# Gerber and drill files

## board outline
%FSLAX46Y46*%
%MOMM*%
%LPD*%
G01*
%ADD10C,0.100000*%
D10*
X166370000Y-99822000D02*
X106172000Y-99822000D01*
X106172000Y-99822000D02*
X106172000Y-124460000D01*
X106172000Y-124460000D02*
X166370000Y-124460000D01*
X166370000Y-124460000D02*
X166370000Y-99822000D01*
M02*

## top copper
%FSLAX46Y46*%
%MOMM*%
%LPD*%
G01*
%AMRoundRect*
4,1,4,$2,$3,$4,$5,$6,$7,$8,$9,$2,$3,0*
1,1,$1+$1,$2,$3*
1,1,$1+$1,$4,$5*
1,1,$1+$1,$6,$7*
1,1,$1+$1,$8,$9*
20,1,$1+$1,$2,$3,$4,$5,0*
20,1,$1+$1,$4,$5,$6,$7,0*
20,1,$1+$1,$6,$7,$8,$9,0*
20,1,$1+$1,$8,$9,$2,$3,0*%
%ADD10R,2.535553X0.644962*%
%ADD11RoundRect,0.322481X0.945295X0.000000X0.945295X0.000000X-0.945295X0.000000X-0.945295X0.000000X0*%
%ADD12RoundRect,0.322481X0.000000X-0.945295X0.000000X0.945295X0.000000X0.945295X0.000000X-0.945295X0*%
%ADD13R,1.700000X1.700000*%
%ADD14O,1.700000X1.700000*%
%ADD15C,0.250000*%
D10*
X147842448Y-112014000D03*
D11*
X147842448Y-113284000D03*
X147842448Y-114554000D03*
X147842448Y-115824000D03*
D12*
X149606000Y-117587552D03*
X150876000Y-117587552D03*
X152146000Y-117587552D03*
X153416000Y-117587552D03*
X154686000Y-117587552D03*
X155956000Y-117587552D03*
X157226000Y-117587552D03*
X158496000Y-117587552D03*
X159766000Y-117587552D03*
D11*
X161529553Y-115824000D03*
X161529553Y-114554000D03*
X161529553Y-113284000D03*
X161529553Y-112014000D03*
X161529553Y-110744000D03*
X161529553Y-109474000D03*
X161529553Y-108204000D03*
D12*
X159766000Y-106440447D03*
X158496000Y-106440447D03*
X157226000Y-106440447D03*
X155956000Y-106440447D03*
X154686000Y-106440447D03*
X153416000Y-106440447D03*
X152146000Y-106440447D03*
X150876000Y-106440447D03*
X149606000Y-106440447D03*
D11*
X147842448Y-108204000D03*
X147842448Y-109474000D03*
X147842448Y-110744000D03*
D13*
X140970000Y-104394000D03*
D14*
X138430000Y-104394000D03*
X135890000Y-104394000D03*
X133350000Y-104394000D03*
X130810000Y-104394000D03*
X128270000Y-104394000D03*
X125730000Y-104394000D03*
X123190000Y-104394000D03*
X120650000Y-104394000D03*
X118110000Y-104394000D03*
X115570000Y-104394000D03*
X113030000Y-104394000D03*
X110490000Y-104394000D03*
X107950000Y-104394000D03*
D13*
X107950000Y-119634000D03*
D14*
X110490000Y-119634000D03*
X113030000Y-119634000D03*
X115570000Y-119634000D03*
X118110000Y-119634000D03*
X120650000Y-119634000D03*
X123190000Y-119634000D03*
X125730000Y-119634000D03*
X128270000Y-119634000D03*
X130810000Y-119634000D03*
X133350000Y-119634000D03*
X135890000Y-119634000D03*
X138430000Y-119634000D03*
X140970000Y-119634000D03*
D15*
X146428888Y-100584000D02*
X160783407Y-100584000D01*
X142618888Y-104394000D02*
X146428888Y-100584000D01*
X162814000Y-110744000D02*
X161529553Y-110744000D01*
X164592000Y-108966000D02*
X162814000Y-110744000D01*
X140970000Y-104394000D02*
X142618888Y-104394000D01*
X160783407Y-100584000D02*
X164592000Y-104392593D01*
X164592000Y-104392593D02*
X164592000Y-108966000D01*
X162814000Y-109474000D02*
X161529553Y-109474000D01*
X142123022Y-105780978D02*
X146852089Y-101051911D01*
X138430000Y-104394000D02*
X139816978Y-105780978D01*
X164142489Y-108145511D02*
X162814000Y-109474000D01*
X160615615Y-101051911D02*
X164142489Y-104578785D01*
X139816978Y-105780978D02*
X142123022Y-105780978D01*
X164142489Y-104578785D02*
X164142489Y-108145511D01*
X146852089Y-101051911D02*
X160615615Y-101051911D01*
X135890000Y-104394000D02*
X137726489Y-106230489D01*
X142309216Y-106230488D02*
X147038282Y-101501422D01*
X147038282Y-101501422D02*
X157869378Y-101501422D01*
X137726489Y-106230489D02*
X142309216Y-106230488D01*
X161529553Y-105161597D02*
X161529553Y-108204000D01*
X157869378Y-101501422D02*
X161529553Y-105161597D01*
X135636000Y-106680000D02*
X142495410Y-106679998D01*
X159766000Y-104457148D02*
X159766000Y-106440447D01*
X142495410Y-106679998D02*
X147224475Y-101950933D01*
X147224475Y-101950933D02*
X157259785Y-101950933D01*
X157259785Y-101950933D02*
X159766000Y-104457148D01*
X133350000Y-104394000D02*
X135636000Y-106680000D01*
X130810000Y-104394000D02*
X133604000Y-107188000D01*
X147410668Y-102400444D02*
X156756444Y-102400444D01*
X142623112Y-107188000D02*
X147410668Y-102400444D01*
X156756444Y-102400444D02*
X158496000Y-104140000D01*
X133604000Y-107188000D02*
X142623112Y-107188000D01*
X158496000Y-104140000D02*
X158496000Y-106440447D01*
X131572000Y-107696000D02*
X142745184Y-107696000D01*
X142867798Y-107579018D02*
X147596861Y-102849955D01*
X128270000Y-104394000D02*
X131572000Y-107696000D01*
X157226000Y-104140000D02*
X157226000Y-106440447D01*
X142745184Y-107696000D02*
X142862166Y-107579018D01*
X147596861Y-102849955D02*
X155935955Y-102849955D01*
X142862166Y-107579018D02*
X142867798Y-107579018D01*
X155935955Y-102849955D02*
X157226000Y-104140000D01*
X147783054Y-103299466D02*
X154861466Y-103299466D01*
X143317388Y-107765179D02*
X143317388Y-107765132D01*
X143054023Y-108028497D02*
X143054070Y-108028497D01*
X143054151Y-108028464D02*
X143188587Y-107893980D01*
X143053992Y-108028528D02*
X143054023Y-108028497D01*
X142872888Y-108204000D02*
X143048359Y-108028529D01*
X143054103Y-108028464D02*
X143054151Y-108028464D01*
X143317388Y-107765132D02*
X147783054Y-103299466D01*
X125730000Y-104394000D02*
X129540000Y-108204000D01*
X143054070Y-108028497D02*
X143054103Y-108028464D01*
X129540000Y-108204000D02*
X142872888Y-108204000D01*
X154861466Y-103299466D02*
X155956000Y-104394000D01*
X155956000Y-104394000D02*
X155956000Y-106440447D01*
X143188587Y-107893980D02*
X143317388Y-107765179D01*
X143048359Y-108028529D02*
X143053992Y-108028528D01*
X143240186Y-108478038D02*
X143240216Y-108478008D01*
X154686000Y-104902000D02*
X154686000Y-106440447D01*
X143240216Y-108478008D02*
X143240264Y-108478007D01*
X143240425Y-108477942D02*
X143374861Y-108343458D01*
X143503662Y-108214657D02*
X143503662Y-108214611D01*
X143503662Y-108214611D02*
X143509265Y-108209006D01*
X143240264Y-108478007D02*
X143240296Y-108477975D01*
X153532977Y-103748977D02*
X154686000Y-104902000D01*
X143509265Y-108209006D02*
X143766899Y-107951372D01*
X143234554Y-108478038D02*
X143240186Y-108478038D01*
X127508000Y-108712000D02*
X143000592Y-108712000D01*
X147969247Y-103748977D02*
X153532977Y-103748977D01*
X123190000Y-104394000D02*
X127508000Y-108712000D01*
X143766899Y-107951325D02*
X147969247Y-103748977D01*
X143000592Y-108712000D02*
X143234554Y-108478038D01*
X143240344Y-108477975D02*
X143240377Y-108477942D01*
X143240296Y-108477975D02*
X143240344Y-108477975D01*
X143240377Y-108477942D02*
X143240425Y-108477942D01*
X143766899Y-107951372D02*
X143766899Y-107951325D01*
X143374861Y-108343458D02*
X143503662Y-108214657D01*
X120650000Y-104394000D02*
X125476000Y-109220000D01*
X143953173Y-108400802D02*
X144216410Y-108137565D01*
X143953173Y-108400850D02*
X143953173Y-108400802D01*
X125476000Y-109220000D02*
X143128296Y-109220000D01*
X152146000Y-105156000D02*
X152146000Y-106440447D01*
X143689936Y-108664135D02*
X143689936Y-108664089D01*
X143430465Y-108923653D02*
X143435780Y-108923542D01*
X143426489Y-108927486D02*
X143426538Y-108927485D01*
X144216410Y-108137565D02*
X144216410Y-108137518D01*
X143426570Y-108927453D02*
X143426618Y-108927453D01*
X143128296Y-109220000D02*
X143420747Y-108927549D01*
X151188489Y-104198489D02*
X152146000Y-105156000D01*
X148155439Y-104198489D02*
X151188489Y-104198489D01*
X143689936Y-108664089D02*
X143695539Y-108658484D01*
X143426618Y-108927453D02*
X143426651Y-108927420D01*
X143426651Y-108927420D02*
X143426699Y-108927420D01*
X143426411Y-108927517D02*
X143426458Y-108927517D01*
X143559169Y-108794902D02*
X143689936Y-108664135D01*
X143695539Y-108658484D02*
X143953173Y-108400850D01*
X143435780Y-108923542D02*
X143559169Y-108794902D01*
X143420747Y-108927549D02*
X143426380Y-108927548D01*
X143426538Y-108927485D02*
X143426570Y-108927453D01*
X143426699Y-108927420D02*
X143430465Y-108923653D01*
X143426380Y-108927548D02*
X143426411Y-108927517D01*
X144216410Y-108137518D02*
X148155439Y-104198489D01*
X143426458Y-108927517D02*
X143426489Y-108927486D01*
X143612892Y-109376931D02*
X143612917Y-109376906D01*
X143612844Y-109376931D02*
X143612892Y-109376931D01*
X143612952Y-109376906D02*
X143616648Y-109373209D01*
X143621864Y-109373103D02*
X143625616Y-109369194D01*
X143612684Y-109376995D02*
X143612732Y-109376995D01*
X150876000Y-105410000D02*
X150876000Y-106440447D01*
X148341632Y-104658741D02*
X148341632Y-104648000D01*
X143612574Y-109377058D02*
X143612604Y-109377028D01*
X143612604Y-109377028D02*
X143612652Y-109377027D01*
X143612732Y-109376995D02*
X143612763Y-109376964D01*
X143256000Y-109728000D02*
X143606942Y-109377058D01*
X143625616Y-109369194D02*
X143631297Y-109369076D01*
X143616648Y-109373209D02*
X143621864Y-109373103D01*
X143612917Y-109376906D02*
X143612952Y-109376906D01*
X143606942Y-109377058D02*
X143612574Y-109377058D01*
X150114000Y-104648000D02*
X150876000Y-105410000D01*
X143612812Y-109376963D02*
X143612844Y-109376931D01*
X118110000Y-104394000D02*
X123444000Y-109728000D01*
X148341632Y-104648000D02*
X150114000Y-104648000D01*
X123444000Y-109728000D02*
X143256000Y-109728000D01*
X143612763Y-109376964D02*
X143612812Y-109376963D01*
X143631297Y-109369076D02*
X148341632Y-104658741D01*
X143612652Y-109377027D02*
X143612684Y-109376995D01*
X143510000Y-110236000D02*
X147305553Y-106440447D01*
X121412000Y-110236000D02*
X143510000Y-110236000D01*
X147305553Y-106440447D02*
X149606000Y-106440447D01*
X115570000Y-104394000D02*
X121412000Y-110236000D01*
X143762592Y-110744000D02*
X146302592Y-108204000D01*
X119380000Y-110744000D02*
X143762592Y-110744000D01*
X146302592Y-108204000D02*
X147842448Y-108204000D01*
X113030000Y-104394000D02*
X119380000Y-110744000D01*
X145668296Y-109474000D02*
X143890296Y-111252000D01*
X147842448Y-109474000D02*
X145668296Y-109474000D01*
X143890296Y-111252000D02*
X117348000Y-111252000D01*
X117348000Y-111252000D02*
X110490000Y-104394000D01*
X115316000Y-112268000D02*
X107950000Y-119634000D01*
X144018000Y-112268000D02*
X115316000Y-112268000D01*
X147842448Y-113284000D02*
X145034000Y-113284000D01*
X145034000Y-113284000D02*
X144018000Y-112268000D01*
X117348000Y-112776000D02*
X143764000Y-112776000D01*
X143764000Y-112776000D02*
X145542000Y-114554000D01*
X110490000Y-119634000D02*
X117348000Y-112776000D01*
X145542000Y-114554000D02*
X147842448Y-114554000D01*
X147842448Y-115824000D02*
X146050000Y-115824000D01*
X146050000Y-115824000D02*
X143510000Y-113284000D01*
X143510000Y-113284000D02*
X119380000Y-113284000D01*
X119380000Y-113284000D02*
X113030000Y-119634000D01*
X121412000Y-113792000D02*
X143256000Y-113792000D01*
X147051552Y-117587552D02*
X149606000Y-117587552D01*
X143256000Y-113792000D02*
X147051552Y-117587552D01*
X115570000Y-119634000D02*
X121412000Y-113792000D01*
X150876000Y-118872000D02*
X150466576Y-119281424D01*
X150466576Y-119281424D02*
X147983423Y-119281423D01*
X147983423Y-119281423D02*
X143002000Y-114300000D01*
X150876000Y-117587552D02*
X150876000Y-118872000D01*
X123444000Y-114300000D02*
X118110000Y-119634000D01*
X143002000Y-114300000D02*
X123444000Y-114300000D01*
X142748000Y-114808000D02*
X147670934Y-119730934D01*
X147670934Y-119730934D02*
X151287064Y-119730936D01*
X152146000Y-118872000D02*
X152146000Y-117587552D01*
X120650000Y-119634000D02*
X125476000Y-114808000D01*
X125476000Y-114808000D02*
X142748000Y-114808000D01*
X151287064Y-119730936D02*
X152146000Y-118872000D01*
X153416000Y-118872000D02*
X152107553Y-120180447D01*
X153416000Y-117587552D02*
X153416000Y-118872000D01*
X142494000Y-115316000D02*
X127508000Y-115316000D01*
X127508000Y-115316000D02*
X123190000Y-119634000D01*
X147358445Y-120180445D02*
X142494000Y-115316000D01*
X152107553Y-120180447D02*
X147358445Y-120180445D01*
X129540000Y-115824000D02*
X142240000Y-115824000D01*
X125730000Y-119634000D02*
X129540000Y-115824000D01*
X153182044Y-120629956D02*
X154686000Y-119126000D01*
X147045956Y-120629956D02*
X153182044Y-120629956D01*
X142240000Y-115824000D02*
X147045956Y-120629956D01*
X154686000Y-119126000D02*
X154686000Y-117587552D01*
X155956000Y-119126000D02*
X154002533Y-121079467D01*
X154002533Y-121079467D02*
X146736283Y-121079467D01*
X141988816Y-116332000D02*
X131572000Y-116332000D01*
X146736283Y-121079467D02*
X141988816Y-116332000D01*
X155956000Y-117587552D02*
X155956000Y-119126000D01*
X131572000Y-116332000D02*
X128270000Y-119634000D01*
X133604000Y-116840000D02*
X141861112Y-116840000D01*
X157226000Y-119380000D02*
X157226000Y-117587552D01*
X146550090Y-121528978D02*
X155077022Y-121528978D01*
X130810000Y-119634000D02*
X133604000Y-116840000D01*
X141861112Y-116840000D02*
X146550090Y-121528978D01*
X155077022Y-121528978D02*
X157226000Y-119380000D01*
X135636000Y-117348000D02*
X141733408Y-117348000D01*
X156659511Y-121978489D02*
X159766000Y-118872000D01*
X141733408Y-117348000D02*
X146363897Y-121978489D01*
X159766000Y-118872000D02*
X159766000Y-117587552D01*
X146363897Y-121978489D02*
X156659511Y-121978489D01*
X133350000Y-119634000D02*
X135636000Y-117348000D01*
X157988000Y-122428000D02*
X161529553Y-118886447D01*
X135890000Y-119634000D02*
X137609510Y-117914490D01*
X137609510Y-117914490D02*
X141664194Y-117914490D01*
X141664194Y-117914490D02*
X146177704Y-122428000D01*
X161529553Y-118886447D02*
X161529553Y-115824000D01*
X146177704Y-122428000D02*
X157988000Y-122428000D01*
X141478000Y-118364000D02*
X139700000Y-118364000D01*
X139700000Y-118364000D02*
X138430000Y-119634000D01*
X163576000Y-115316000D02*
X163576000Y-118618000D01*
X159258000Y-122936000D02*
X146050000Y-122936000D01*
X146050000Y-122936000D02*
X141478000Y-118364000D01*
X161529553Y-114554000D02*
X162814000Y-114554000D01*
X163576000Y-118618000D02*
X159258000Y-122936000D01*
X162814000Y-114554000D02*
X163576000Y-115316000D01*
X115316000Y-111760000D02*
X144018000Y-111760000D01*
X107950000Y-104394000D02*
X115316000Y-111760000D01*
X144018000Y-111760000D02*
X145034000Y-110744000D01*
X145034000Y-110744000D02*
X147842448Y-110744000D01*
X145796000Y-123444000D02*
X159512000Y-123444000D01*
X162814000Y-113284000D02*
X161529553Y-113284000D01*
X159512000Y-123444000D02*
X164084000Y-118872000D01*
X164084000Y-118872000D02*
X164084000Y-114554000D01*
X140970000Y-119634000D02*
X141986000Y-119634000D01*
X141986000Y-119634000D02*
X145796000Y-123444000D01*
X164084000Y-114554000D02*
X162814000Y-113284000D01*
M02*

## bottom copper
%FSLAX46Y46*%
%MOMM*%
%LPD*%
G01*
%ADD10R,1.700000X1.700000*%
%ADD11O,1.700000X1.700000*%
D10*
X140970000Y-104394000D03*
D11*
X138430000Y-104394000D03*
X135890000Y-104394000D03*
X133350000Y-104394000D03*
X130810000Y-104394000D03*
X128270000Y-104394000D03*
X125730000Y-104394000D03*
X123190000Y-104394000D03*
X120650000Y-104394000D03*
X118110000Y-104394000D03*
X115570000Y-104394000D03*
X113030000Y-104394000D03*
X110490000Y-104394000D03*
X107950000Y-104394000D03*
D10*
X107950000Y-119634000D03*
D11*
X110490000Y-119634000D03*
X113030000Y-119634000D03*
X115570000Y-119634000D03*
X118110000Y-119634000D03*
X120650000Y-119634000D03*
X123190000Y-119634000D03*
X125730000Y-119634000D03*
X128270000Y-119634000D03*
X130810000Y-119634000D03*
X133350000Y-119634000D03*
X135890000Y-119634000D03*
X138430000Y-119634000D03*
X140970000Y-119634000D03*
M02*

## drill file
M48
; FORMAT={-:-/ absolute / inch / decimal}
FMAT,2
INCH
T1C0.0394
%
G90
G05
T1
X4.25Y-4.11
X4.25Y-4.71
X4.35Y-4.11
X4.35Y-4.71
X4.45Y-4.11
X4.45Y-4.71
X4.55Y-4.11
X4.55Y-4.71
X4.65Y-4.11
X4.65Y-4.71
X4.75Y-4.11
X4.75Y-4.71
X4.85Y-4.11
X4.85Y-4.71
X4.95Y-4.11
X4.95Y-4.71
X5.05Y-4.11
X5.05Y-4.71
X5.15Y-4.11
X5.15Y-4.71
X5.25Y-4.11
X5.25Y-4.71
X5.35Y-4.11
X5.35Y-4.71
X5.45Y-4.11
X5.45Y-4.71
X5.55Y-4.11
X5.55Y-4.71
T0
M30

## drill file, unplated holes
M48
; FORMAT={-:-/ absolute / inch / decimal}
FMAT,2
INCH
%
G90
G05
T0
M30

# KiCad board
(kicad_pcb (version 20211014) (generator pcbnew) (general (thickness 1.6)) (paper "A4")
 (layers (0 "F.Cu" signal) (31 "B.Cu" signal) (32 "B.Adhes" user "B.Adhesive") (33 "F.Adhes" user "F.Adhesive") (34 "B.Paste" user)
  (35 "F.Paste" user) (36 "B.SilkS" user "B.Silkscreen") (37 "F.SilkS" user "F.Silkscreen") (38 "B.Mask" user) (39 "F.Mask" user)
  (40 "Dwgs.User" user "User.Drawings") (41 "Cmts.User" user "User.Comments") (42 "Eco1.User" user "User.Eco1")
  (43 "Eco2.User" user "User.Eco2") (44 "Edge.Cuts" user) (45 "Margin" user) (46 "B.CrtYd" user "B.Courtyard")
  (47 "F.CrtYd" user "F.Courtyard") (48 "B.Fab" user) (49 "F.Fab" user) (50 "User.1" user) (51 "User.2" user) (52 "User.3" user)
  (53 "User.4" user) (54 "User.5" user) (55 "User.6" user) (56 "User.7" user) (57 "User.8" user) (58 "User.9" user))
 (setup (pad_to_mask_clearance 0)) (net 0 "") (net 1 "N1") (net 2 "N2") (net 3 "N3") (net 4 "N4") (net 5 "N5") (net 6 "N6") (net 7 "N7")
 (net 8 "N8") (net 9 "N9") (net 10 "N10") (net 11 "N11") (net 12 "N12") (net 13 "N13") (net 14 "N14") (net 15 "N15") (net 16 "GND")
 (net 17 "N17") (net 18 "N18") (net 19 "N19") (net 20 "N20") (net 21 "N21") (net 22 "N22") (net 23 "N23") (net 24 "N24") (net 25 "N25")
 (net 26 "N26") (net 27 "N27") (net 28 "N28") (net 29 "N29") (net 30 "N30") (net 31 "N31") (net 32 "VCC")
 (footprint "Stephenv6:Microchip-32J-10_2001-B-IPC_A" (layer "F.Cu") (at 154.686 112.014 90)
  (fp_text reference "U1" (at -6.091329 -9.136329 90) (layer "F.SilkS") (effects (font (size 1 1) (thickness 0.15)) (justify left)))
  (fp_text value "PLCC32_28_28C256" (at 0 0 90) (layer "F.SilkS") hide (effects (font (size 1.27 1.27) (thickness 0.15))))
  (pad "1" smd rect (at 0 -6.843552 90) (size 0.644962 2.535553) (layers "F.Cu" "F.Paste" "F.Mask") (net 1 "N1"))
  (pad "2" smd roundrect (at -1.27 -6.843552 90) (size 0.644962 2.535553) (layers "F.Cu" "F.Paste" "F.Mask") (roundrect_rratio 0.5)
   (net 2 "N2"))
  (pad "3" smd roundrect (at -2.54 -6.843552 90) (size 0.644962 2.535553) (layers "F.Cu" "F.Paste" "F.Mask") (roundrect_rratio 0.5)
   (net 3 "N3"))
  (pad "4" smd roundrect (at -3.81 -6.843552 90) (size 0.644962 2.535553) (layers "F.Cu" "F.Paste" "F.Mask") (roundrect_rratio 0.5)
   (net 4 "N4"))
  (pad "5" smd roundrect (at -5.573552 -5.08 90) (size 2.535553 0.644962) (layers "F.Cu" "F.Paste" "F.Mask") (roundrect_rratio 0.5)
   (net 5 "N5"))
  (pad "6" smd roundrect (at -5.573552 -3.81 90) (size 2.535553 0.644962) (layers "F.Cu" "F.Paste" "F.Mask") (roundrect_rratio 0.5)
   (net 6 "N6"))
  (pad "7" smd roundrect (at -5.573552 -2.54 90) (size 2.535553 0.644962) (layers "F.Cu" "F.Paste" "F.Mask") (roundrect_rratio 0.5)
   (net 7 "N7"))
  (pad "8" smd roundrect (at -5.573552 -1.27 90) (size 2.535553 0.644962) (layers "F.Cu" "F.Paste" "F.Mask") (roundrect_rratio 0.5)
   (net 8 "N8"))
  (pad "9" smd roundrect (at -5.573552 0 90) (size 2.535553 0.644962) (layers "F.Cu" "F.Paste" "F.Mask") (roundrect_rratio 0.5) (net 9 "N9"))
  (pad "10" smd roundrect (at -5.573552 1.27 90) (size 2.535553 0.644962) (layers "F.Cu" "F.Paste" "F.Mask") (roundrect_rratio 0.5)
   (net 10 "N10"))
  (pad "11" smd roundrect (at -5.573552 2.54 90) (size 2.535553 0.644962) (layers "F.Cu" "F.Paste" "F.Mask") (roundrect_rratio 0.5)
   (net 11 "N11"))
  (pad "12" smd roundrect (at -5.573552 3.81 90) (size 2.535553 0.644962) (layers "F.Cu" "F.Paste" "F.Mask") (roundrect_rratio 0.5)
   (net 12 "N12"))
  (pad "13" smd roundrect (at -5.573552 5.08 90) (size 2.535553 0.644962) (layers "F.Cu" "F.Paste" "F.Mask") (roundrect_rratio 0.5)
   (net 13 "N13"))
  (pad "14" smd roundrect (at -3.81 6.843553 90) (size 0.644962 2.535553) (layers "F.Cu" "F.Paste" "F.Mask") (roundrect_rratio 0.5)
   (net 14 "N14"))
  (pad "15" smd roundrect (at -2.54 6.843553 90) (size 0.644962 2.535553) (layers "F.Cu" "F.Paste" "F.Mask") (roundrect_rratio 0.5)
   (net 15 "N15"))
  (pad "16" smd roundrect (at -1.27 6.843553 90) (size 0.644962 2.535553) (layers "F.Cu" "F.Paste" "F.Mask") (roundrect_rratio 0.5)
   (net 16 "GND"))
  (pad "17" smd roundrect (at 0 6.843553 90) (size 0.644962 2.535553) (layers "F.Cu" "F.Paste" "F.Mask") (roundrect_rratio 0.5)
   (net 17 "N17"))
  (pad "18" smd roundrect (at 1.27 6.843553 90) (size 0.644962 2.535553) (layers "F.Cu" "F.Paste" "F.Mask") (roundrect_rratio 0.5)
   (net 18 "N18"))
  (pad "19" smd roundrect (at 2.54 6.843553 90) (size 0.644962 2.535553) (layers "F.Cu" "F.Paste" "F.Mask") (roundrect_rratio 0.5)
   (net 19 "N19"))
  (pad "20" smd roundrect (at 3.81 6.843553 90) (size 0.644962 2.535553) (layers "F.Cu" "F.Paste" "F.Mask") (roundrect_rratio 0.5)
   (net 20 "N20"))
  (pad "21" smd roundrect (at 5.573553 5.08 90) (size 2.535553 0.644962) (layers "F.Cu" "F.Paste" "F.Mask") (roundrect_rratio 0.5)
   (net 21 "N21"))
  (pad "22" smd roundrect (at 5.573553 3.81 90) (size 2.535553 0.644962) (layers "F.Cu" "F.Paste" "F.Mask") (roundrect_rratio 0.5)
   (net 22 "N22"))
  (pad "23" smd roundrect (at 5.573553 2.54 90) (size 2.535553 0.644962) (layers "F.Cu" "F.Paste" "F.Mask") (roundrect_rratio 0.5)
   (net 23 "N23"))
  (pad "24" smd roundrect (at 5.573553 1.27 90) (size 2.535553 0.644962) (layers "F.Cu" "F.Paste" "F.Mask") (roundrect_rratio 0.5)
   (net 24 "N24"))
  (pad "25" smd roundrect (at 5.573553 0 90) (size 2.535553 0.644962) (layers "F.Cu" "F.Paste" "F.Mask") (roundrect_rratio 0.5)
   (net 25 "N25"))
  (pad "26" smd roundrect (at 5.573553 -1.27 90) (size 2.535553 0.644962) (layers "F.Cu" "F.Paste" "F.Mask") (roundrect_rratio 0.5)
   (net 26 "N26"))
  (pad "27" smd roundrect (at 5.573553 -2.54 90) (size 2.535553 0.644962) (layers "F.Cu" "F.Paste" "F.Mask") (roundrect_rratio 0.5)
   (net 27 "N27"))
  (pad "28" smd roundrect (at 5.573553 -3.81 90) (size 2.535553 0.644962) (layers "F.Cu" "F.Paste" "F.Mask") (roundrect_rratio 0.5)
   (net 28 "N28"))
  (pad "29" smd roundrect (at 5.573553 -5.08 90) (size 2.535553 0.644962) (layers "F.Cu" "F.Paste" "F.Mask") (roundrect_rratio 0.5)
   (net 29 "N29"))
  (pad "30" smd roundrect (at 3.81 -6.843552 90) (size 0.644962 2.535553) (layers "F.Cu" "F.Paste" "F.Mask") (roundrect_rratio 0.5)
   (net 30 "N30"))
  (pad "31" smd roundrect (at 2.54 -6.843552 90) (size 0.644962 2.535553) (layers "F.Cu" "F.Paste" "F.Mask") (roundrect_rratio 0.5)
   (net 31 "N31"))
  (pad "32" smd roundrect (at 1.27 -6.843552 90) (size 0.644962 2.535553) (layers "F.Cu" "F.Paste" "F.Mask") (roundrect_rratio 0.5)
   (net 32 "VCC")))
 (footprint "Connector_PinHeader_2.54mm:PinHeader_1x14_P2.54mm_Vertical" (layer "B.Cu") (at 140.97 104.394 90)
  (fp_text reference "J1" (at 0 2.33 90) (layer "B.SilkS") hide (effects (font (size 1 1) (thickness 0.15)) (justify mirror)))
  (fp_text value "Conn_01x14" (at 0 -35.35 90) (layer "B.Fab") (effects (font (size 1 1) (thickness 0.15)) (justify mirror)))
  (pad "1" thru_hole rect locked (at 0 0 90) (size 1.7 1.7) (drill 1) (layers *.Cu *.Mask) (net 18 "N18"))
  (pad "2" thru_hole oval locked (at 0 -2.54 90) (size 1.7 1.7) (drill 1) (layers *.Cu *.Mask) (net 19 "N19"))
  (pad "3" thru_hole oval locked (at 0 -5.08 90) (size 1.7 1.7) (drill 1) (layers *.Cu *.Mask) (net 20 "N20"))
  (pad "4" thru_hole oval locked (at 0 -7.62 90) (size 1.7 1.7) (drill 1) (layers *.Cu *.Mask) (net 21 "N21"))
  (pad "5" thru_hole oval locked (at 0 -10.16 90) (size 1.7 1.7) (drill 1) (layers *.Cu *.Mask) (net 22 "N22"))
  (pad "6" thru_hole oval locked (at 0 -12.7 90) (size 1.7 1.7) (drill 1) (layers *.Cu *.Mask) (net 23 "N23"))
  (pad "7" thru_hole oval locked (at 0 -15.24 90) (size 1.7 1.7) (drill 1) (layers *.Cu *.Mask) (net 24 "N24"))
  (pad "8" thru_hole oval locked (at 0 -17.78 90) (size 1.7 1.7) (drill 1) (layers *.Cu *.Mask) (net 25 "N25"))
  (pad "9" thru_hole oval locked (at 0 -20.32 90) (size 1.7 1.7) (drill 1) (layers *.Cu *.Mask) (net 27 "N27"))
  (pad "10" thru_hole oval locked (at 0 -22.86 90) (size 1.7 1.7) (drill 1) (layers *.Cu *.Mask) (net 28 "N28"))
  (pad "11" thru_hole oval locked (at 0 -25.4 90) (size 1.7 1.7) (drill 1) (layers *.Cu *.Mask) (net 29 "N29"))
  (pad "12" thru_hole oval locked (at 0 -27.94 90) (size 1.7 1.7) (drill 1) (layers *.Cu *.Mask) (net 30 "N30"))
  (pad "13" thru_hole oval locked (at 0 -30.48 90) (size 1.7 1.7) (drill 1) (layers *.Cu *.Mask) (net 31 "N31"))
  (pad "14" thru_hole oval locked (at 0 -33.02 90) (size 1.7 1.7) (drill 1) (layers *.Cu *.Mask) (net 32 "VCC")))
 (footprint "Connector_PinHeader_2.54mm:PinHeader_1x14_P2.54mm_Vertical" (layer "B.Cu") (at 107.95 119.634 -90)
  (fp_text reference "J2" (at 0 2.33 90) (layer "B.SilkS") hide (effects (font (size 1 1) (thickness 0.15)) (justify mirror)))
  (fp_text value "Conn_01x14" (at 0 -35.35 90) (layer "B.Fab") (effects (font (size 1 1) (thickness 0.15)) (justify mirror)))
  (pad "1" thru_hole rect locked (at 0 0 270) (size 1.7 1.7) (drill 1) (layers *.Cu *.Mask) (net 2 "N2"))
  (pad "2" thru_hole oval locked (at 0 -2.54 270) (size 1.7 1.7) (drill 1) (layers *.Cu *.Mask) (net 3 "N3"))
  (pad "3" thru_hole oval locked (at 0 -5.08 270) (size 1.7 1.7) (drill 1) (layers *.Cu *.Mask) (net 4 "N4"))
  (pad "4" thru_hole oval locked (at 0 -7.62 270) (size 1.7 1.7) (drill 1) (layers *.Cu *.Mask) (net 5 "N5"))
  (pad "5" thru_hole oval locked (at 0 -10.16 270) (size 1.7 1.7) (drill 1) (layers *.Cu *.Mask) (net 6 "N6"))
  (pad "6" thru_hole oval locked (at 0 -12.7 270) (size 1.7 1.7) (drill 1) (layers *.Cu *.Mask) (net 7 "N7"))
  (pad "7" thru_hole oval locked (at 0 -15.24 270) (size 1.7 1.7) (drill 1) (layers *.Cu *.Mask) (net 8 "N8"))
  (pad "8" thru_hole oval locked (at 0 -17.78 270) (size 1.7 1.7) (drill 1) (layers *.Cu *.Mask) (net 9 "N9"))
  (pad "9" thru_hole oval locked (at 0 -20.32 270) (size 1.7 1.7) (drill 1) (layers *.Cu *.Mask) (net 10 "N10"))
  (pad "10" thru_hole oval locked (at 0 -22.86 270) (size 1.7 1.7) (drill 1) (layers *.Cu *.Mask) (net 11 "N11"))
  (pad "11" thru_hole oval locked (at 0 -25.4 270) (size 1.7 1.7) (drill 1) (layers *.Cu *.Mask) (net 13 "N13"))
  (pad "12" thru_hole oval locked (at 0 -27.94 270) (size 1.7 1.7) (drill 1) (layers *.Cu *.Mask) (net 14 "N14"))
  (pad "13" thru_hole oval locked (at 0 -30.48 270) (size 1.7 1.7) (drill 1) (layers *.Cu *.Mask) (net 15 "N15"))
  (pad "14" thru_hole oval locked (at 0 -33.02 270) (size 1.7 1.7) (drill 1) (layers *.Cu *.Mask) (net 16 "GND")))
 (gr_rect (start 166.37 99.822) (end 106.172 124.46) (layer "Edge.Cuts") (width 0.1) (fill none))
 (segment (start 146.428888 100.584) (end 160.783407 100.584) (width 0.25) (layer "F.Cu") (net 18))
 (segment (start 142.618888 104.394) (end 146.428888 100.584) (width 0.25) (layer "F.Cu") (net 18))
 (segment (start 162.814 110.744) (end 161.529553 110.744) (width 0.25) (layer "F.Cu") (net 18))
 (segment (start 164.592 108.966) (end 162.814 110.744) (width 0.25) (layer "F.Cu") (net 18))
 (segment (start 140.97 104.394) (end 142.618888 104.394) (width 0.25) (layer "F.Cu") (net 18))
 (segment (start 160.783407 100.584) (end 164.592 104.392593) (width 0.25) (layer "F.Cu") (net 18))
 (segment (start 164.592 104.392593) (end 164.592 108.966) (width 0.25) (layer "F.Cu") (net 18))
 (segment (start 162.814 109.474) (end 161.529553 109.474) (width 0.25) (layer "F.Cu") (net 19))
 (segment (start 142.123022 105.780978) (end 146.852089 101.051911) (width 0.25) (layer "F.Cu") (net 19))
 (segment (start 138.43 104.394) (end 139.816978 105.780978) (width 0.25) (layer "F.Cu") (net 19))
 (segment (start 164.142489 108.145511) (end 162.814 109.474) (width 0.25) (layer "F.Cu") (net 19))
 (segment (start 160.615615 101.051911) (end 164.142489 104.578785) (width 0.25) (layer "F.Cu") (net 19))
 (segment (start 139.816978 105.780978) (end 142.123022 105.780978) (width 0.25) (layer "F.Cu") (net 19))
 (segment (start 164.142489 104.578785) (end 164.142489 108.145511) (width 0.25) (layer "F.Cu") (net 19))
 (segment (start 146.852089 101.051911) (end 160.615615 101.051911) (width 0.25) (layer "F.Cu") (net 19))
 (segment (start 135.89 104.394) (end 137.726489 106.230489) (width 0.25) (layer "F.Cu") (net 20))
 (segment (start 142.309216 106.230488) (end 147.038282 101.501422) (width 0.25) (layer "F.Cu") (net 20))
 (segment (start 147.038282 101.501422) (end 157.869378 101.501422) (width 0.25) (layer "F.Cu") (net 20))
 (segment (start 137.726489 106.230489) (end 142.309216 106.230488) (width 0.25) (layer "F.Cu") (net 20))
 (segment (start 161.529553 105.161597) (end 161.529553 108.204) (width 0.25) (layer "F.Cu") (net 20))
 (segment (start 157.869378 101.501422) (end 161.529553 105.161597) (width 0.25) (layer "F.Cu") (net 20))
 (segment (start 135.636 106.68) (end 142.49541 106.679998) (width 0.25) (layer "F.Cu") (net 21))
 (segment (start 159.766 104.457148) (end 159.766 106.440447) (width 0.25) (layer "F.Cu") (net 21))
 (segment (start 142.49541 106.679998) (end 147.224475 101.950933) (width 0.25) (layer "F.Cu") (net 21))
 (segment (start 147.224475 101.950933) (end 157.259785 101.950933) (width 0.25) (layer "F.Cu") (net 21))
 (segment (start 157.259785 101.950933) (end 159.766 104.457148) (width 0.25) (layer "F.Cu") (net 21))
 (segment (start 133.35 104.394) (end 135.636 106.68) (width 0.25) (layer "F.Cu") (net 21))
 (segment (start 130.81 104.394) (end 133.604 107.188) (width 0.25) (layer "F.Cu") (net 22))
 (segment (start 147.410668 102.400444) (end 156.756444 102.400444) (width 0.25) (layer "F.Cu") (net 22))
 (segment (start 142.623112 107.188) (end 147.410668 102.400444) (width 0.25) (layer "F.Cu") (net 22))
 (segment (start 156.756444 102.400444) (end 158.496 104.14) (width 0.25) (layer "F.Cu") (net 22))
 (segment (start 133.604 107.188) (end 142.623112 107.188) (width 0.25) (layer "F.Cu") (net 22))
 (segment (start 158.496 104.14) (end 158.496 106.440447) (width 0.25) (layer "F.Cu") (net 22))
 (segment (start 131.572 107.696) (end 142.745184 107.696) (width 0.25) (layer "F.Cu") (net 23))
 (segment (start 142.867798 107.579018) (end 147.596861 102.849955) (width 0.25) (layer "F.Cu") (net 23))
 (segment (start 128.27 104.394) (end 131.572 107.696) (width 0.25) (layer "F.Cu") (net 23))
 (segment (start 157.226 104.14) (end 157.226 106.440447) (width 0.25) (layer "F.Cu") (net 23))
 (segment (start 142.745184 107.696) (end 142.862166 107.579018) (width 0.25) (layer "F.Cu") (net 23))
 (segment (start 147.596861 102.849955) (end 155.935955 102.849955) (width 0.25) (layer "F.Cu") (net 23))
 (segment (start 142.862166 107.579018) (end 142.867798 107.579018) (width 0.25) (layer "F.Cu") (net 23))
 (segment (start 155.935955 102.849955) (end 157.226 104.14) (width 0.25) (layer "F.Cu") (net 23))
 (segment (start 147.783054 103.299466) (end 154.861466 103.299466) (width 0.25) (layer "F.Cu") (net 24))
 (segment (start 143.317388 107.765179) (end 143.317388 107.765132) (width 0.25) (layer "F.Cu") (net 24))
 (segment (start 143.054023 108.028497) (end 143.05407 108.028497) (width 0.25) (layer "F.Cu") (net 24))
 (segment (start 143.054151 108.028464) (end 143.188587 107.89398) (width 0.25) (layer "F.Cu") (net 24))
 (segment (start 143.053992 108.028528) (end 143.054023 108.028497) (width 0.25) (layer "F.Cu") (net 24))
 (segment (start 142.872888 108.204) (end 143.048359 108.028529) (width 0.25) (layer "F.Cu") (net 24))
 (segment (start 143.054103 108.028464) (end 143.054151 108.028464) (width 0.25) (layer "F.Cu") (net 24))
 (segment (start 143.317388 107.765132) (end 147.783054 103.299466) (width 0.25) (layer "F.Cu") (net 24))
 (segment (start 125.73 104.394) (end 129.54 108.204) (width 0.25) (layer "F.Cu") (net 24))
 (segment (start 143.05407 108.028497) (end 143.054103 108.028464) (width 0.25) (layer "F.Cu") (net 24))
 (segment (start 129.54 108.204) (end 142.872888 108.204) (width 0.25) (layer "F.Cu") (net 24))
 (segment (start 154.861466 103.299466) (end 155.956 104.394) (width 0.25) (layer "F.Cu") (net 24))
 (segment (start 155.956 104.394) (end 155.956 106.440447) (width 0.25) (layer "F.Cu") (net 24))
 (segment (start 143.188587 107.89398) (end 143.317388 107.765179) (width 0.25) (layer "F.Cu") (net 24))
 (segment (start 143.048359 108.028529) (end 143.053992 108.028528) (width 0.25) (layer "F.Cu") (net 24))
 (segment (start 143.240186 108.478038) (end 143.240216 108.478008) (width 0.25) (layer "F.Cu") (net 25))
 (segment (start 154.686 104.902) (end 154.686 106.440447) (width 0.25) (layer "F.Cu") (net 25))
 (segment (start 143.240216 108.478008) (end 143.240264 108.478007) (width 0.25) (layer "F.Cu") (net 25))
 (segment (start 143.240425 108.477942) (end 143.374861 108.343458) (width 0.25) (layer "F.Cu") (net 25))
 (segment (start 143.503662 108.214657) (end 143.503662 108.214611) (width 0.25) (layer "F.Cu") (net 25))
 (segment (start 143.503662 108.214611) (end 143.509265 108.209006) (width 0.25) (layer "F.Cu") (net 25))
 (segment (start 143.240264 108.478007) (end 143.240296 108.477975) (width 0.25) (layer "F.Cu") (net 25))
 (segment (start 153.532977 103.748977) (end 154.686 104.902) (width 0.25) (layer "F.Cu") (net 25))
 (segment (start 143.509265 108.209006) (end 143.766899 107.951372) (width 0.25) (layer "F.Cu") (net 25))
 (segment (start 143.234554 108.478038) (end 143.240186 108.478038) (width 0.25) (layer "F.Cu") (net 25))
 (segment (start 127.508 108.712) (end 143.000592 108.712) (width 0.25) (layer "F.Cu") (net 25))
 (segment (start 147.969247 103.748977) (end 153.532977 103.748977) (width 0.25) (layer "F.Cu") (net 25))
 (segment (start 123.19 104.394) (end 127.508 108.712) (width 0.25) (layer "F.Cu") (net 25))
 (segment (start 143.766899 107.951325) (end 147.969247 103.748977) (width 0.25) (layer "F.Cu") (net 25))
 (segment (start 143.000592 108.712) (end 143.234554 108.478038) (width 0.25) (layer "F.Cu") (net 25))
 (segment (start 143.240344 108.477975) (end 143.240377 108.477942) (width 0.25) (layer "F.Cu") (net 25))
 (segment (start 143.240296 108.477975) (end 143.240344 108.477975) (width 0.25) (layer "F.Cu") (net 25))
 (segment (start 143.240377 108.477942) (end 143.240425 108.477942) (width 0.25) (layer "F.Cu") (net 25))
 (segment (start 143.766899 107.951372) (end 143.766899 107.951325) (width 0.25) (layer "F.Cu") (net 25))
 (segment (start 143.374861 108.343458) (end 143.503662 108.214657) (width 0.25) (layer "F.Cu") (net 25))
 (segment (start 120.65 104.394) (end 125.476 109.22) (width 0.25) (layer "F.Cu") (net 27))
 (segment (start 143.953173 108.400802) (end 144.21641 108.137565) (width 0.25) (layer "F.Cu") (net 27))
 (segment (start 143.953173 108.40085) (end 143.953173 108.400802) (width 0.25) (layer "F.Cu") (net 27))
 (segment (start 125.476 109.22) (end 143.128296 109.22) (width 0.25) (layer "F.Cu") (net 27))
 (segment (start 152.146 105.156) (end 152.146 106.440447) (width 0.25) (layer "F.Cu") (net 27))
 (segment (start 143.689936 108.664135) (end 143.689936 108.664089) (width 0.25) (layer "F.Cu") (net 27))
 (segment (start 143.430465 108.923653) (end 143.43578 108.923542) (width 0.25) (layer "F.Cu") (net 27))
 (segment (start 143.426489 108.927486) (end 143.426538 108.927485) (width 0.25) (layer "F.Cu") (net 27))
 (segment (start 144.21641 108.137565) (end 144.21641 108.137518) (width 0.25) (layer "F.Cu") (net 27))
 (segment (start 143.42657 108.927453) (end 143.426618 108.927453) (width 0.25) (layer "F.Cu") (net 27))
 (segment (start 143.128296 109.22) (end 143.420747 108.927549) (width 0.25) (layer "F.Cu") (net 27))
 (segment (start 151.188489 104.198489) (end 152.146 105.156) (width 0.25) (layer "F.Cu") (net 27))
 (segment (start 148.155439 104.198489) (end 151.188489 104.198489) (width 0.25) (layer "F.Cu") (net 27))
 (segment (start 143.689936 108.664089) (end 143.695539 108.658484) (width 0.25) (layer "F.Cu") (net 27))
 (segment (start 143.426618 108.927453) (end 143.426651 108.92742) (width 0.25) (layer "F.Cu") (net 27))
 (segment (start 143.426651 108.92742) (end 143.426699 108.92742) (width 0.25) (layer "F.Cu") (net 27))
 (segment (start 143.426411 108.927517) (end 143.426458 108.927517) (width 0.25) (layer "F.Cu") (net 27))
 (segment (start 143.559169 108.794902) (end 143.689936 108.664135) (width 0.25) (layer "F.Cu") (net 27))
 (segment (start 143.695539 108.658484) (end 143.953173 108.40085) (width 0.25) (layer "F.Cu") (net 27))
 (segment (start 143.43578 108.923542) (end 143.559169 108.794902) (width 0.25) (layer "F.Cu") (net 27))
 (segment (start 143.420747 108.927549) (end 143.42638 108.927548) (width 0.25) (layer "F.Cu") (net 27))
 (segment (start 143.426538 108.927485) (end 143.42657 108.927453) (width 0.25) (layer "F.Cu") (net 27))
 (segment (start 143.426699 108.92742) (end 143.430465 108.923653) (width 0.25) (layer "F.Cu") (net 27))
 (segment (start 143.42638 108.927548) (end 143.426411 108.927517) (width 0.25) (layer "F.Cu") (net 27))
 (segment (start 144.21641 108.137518) (end 148.155439 104.198489) (width 0.25) (layer "F.Cu") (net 27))
 (segment (start 143.426458 108.927517) (end 143.426489 108.927486) (width 0.25) (layer "F.Cu") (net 27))
 (segment (start 143.612892 109.376931) (end 143.612917 109.376906) (width 0.25) (layer "F.Cu") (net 28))
 (segment (start 143.612844 109.376931) (end 143.612892 109.376931) (width 0.25) (layer "F.Cu") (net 28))
 (segment (start 143.612952 109.376906) (end 143.616648 109.373209) (width 0.25) (layer "F.Cu") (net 28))
 (segment (start 143.621864 109.373103) (end 143.625616 109.369194) (width 0.25) (layer "F.Cu") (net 28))
 (segment (start 143.612684 109.376995) (end 143.612732 109.376995) (width 0.25) (layer "F.Cu") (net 28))
 (segment (start 150.876 105.41) (end 150.876 106.440447) (width 0.25) (layer "F.Cu") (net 28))
 (segment (start 148.341632 104.658741) (end 148.341632 104.648) (width 0.25) (layer "F.Cu") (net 28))
 (segment (start 143.612574 109.377058) (end 143.612604 109.377028) (width 0.25) (layer "F.Cu") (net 28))
 (segment (start 143.612604 109.377028) (end 143.612652 109.377027) (width 0.25) (layer "F.Cu") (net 28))
 (segment (start 143.612732 109.376995) (end 143.612763 109.376964) (width 0.25) (layer "F.Cu") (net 28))
 (segment (start 143.256 109.728) (end 143.606942 109.377058) (width 0.25) (layer "F.Cu") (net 28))
 (segment (start 143.625616 109.369194) (end 143.631297 109.369076) (width 0.25) (layer "F.Cu") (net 28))
 (segment (start 143.616648 109.373209) (end 143.621864 109.373103) (width 0.25) (layer "F.Cu") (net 28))
 (segment (start 143.612917 109.376906) (end 143.612952 109.376906) (width 0.25) (layer "F.Cu") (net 28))
 (segment (start 143.606942 109.377058) (end 143.612574 109.377058) (width 0.25) (layer "F.Cu") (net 28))
 (segment (start 150.114 104.648) (end 150.876 105.41) (width 0.25) (layer "F.Cu") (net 28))
 (segment (start 143.612812 109.376963) (end 143.612844 109.376931) (width 0.25) (layer "F.Cu") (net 28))
 (segment (start 118.11 104.394) (end 123.444 109.728) (width 0.25) (layer "F.Cu") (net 28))
 (segment (start 148.341632 104.648) (end 150.114 104.648) (width 0.25) (layer "F.Cu") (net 28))
 (segment (start 123.444 109.728) (end 143.256 109.728) (width 0.25) (layer "F.Cu") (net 28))
 (segment (start 143.612763 109.376964) (end 143.612812 109.376963) (width 0.25) (layer "F.Cu") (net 28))
 (segment (start 143.631297 109.369076) (end 148.341632 104.658741) (width 0.25) (layer "F.Cu") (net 28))
 (segment (start 143.612652 109.377027) (end 143.612684 109.376995) (width 0.25) (layer "F.Cu") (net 28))
 (segment (start 143.51 110.236) (end 147.305553 106.440447) (width 0.25) (layer "F.Cu") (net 29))
 (segment (start 121.412 110.236) (end 143.51 110.236) (width 0.25) (layer "F.Cu") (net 29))
 (segment (start 147.305553 106.440447) (end 149.606 106.440447) (width 0.25) (layer "F.Cu") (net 29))
 (segment (start 115.57 104.394) (end 121.412 110.236) (width 0.25) (layer "F.Cu") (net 29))
 (segment (start 143.762592 110.744) (end 146.302592 108.204) (width 0.25) (layer "F.Cu") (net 30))
 (segment (start 119.38 110.744) (end 143.762592 110.744) (width 0.25) (layer "F.Cu") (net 30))
 (segment (start 146.302592 108.204) (end 147.842448 108.204) (width 0.25) (layer "F.Cu") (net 30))
 (segment (start 113.03 104.394) (end 119.38 110.744) (width 0.25) (layer "F.Cu") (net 30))
 (segment (start 145.668296 109.474) (end 143.890296 111.252) (width 0.25) (layer "F.Cu") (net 31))
 (segment (start 147.842448 109.474) (end 145.668296 109.474) (width 0.25) (layer "F.Cu") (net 31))
 (segment (start 143.890296 111.252) (end 117.348 111.252) (width 0.25) (layer "F.Cu") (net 31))
 (segment (start 117.348 111.252) (end 110.49 104.394) (width 0.25) (layer "F.Cu") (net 31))
 (segment (start 115.316 112.268) (end 107.95 119.634) (width 0.25) (layer "F.Cu") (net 2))
 (segment (start 144.018 112.268) (end 115.316 112.268) (width 0.25) (layer "F.Cu") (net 2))
 (segment (start 147.842448 113.284) (end 145.034 113.284) (width 0.25) (layer "F.Cu") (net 2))
 (segment (start 145.034 113.284) (end 144.018 112.268) (width 0.25) (layer "F.Cu") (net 2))
 (segment (start 117.348 112.776) (end 143.764 112.776) (width 0.25) (layer "F.Cu") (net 3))
 (segment (start 143.764 112.776) (end 145.542 114.554) (width 0.25) (layer "F.Cu") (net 3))
 (segment (start 110.49 119.634) (end 117.348 112.776) (width 0.25) (layer "F.Cu") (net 3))
 (segment (start 145.542 114.554) (end 147.842448 114.554) (width 0.25) (layer "F.Cu") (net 3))
 (segment (start 147.842448 115.824) (end 146.05 115.824) (width 0.25) (layer "F.Cu") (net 4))
 (segment (start 146.05 115.824) (end 143.51 113.284) (width 0.25) (layer "F.Cu") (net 4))
 (segment (start 143.51 113.284) (end 119.38 113.284) (width 0.25) (layer "F.Cu") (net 4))
 (segment (start 119.38 113.284) (end 113.03 119.634) (width 0.25) (layer "F.Cu") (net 4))
 (segment (start 121.412 113.792) (end 143.256 113.792) (width 0.25) (layer "F.Cu") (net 5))
 (segment (start 147.051552 117.587552) (end 149.606 117.587552) (width 0.25) (layer "F.Cu") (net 5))
 (segment (start 143.256 113.792) (end 147.051552 117.587552) (width 0.25) (layer "F.Cu") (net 5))
 (segment (start 115.57 119.634) (end 121.412 113.792) (width 0.25) (layer "F.Cu") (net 5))
 (segment (start 150.876 118.872) (end 150.466576 119.281424) (width 0.25) (layer "F.Cu") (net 6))
 (segment (start 150.466576 119.281424) (end 147.983423 119.281423) (width 0.25) (layer "F.Cu") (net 6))
 (segment (start 147.983423 119.281423) (end 143.002 114.3) (width 0.25) (layer "F.Cu") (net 6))
 (segment (start 150.876 117.587552) (end 150.876 118.872) (width 0.25) (layer "F.Cu") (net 6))
 (segment (start 123.444 114.3) (end 118.11 119.634) (width 0.25) (layer "F.Cu") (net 6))
 (segment (start 143.002 114.3) (end 123.444 114.3) (width 0.25) (layer "F.Cu") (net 6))
 (segment (start 142.748 114.808) (end 147.670934 119.730934) (width 0.25) (layer "F.Cu") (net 7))
 (segment (start 147.670934 119.730934) (end 151.287064 119.730936) (width 0.25) (layer "F.Cu") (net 7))
 (segment (start 152.146 118.872) (end 152.146 117.587552) (width 0.25) (layer "F.Cu") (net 7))
 (segment (start 120.65 119.634) (end 125.476 114.808) (width 0.25) (layer "F.Cu") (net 7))
 (segment (start 125.476 114.808) (end 142.748 114.808) (width 0.25) (layer "F.Cu") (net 7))
 (segment (start 151.287064 119.730936) (end 152.146 118.872) (width 0.25) (layer "F.Cu") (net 7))
 (segment (start 153.416 118.872) (end 152.107553 120.180447) (width 0.25) (layer "F.Cu") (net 8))
 (segment (start 153.416 117.587552) (end 153.416 118.872) (width 0.25) (layer "F.Cu") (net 8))
 (segment (start 142.494 115.316) (end 127.508 115.316) (width 0.25) (layer "F.Cu") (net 8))
 (segment (start 127.508 115.316) (end 123.19 119.634) (width 0.25) (layer "F.Cu") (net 8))
 (segment (start 147.358445 120.180445) (end 142.494 115.316) (width 0.25) (layer "F.Cu") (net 8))
 (segment (start 152.107553 120.180447) (end 147.358445 120.180445) (width 0.25) (layer "F.Cu") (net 8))
 (segment (start 129.54 115.824) (end 142.24 115.824) (width 0.25) (layer "F.Cu") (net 9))
 (segment (start 125.73 119.634) (end 129.54 115.824) (width 0.25) (layer "F.Cu") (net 9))
 (segment (start 153.182044 120.629956) (end 154.686 119.126) (width 0.25) (layer "F.Cu") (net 9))
 (segment (start 147.045956 120.629956) (end 153.182044 120.629956) (width 0.25) (layer "F.Cu") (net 9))
 (segment (start 142.24 115.824) (end 147.045956 120.629956) (width 0.25) (layer "F.Cu") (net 9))
 (segment (start 154.686 119.126) (end 154.686 117.587552) (width 0.25) (layer "F.Cu") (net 9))
 (segment (start 155.956 119.126) (end 154.002533 121.079467) (width 0.25) (layer "F.Cu") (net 10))
 (segment (start 154.002533 121.079467) (end 146.736283 121.079467) (width 0.25) (layer "F.Cu") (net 10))
 (segment (start 141.988816 116.332) (end 131.572 116.332) (width 0.25) (layer "F.Cu") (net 10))
 (segment (start 146.736283 121.079467) (end 141.988816 116.332) (width 0.25) (layer "F.Cu") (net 10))
 (segment (start 155.956 117.587552) (end 155.956 119.126) (width 0.25) (layer "F.Cu") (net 10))
 (segment (start 131.572 116.332) (end 128.27 119.634) (width 0.25) (layer "F.Cu") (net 10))
 (segment (start 133.604 116.84) (end 141.861112 116.84) (width 0.25) (layer "F.Cu") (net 11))
 (segment (start 157.226 119.38) (end 157.226 117.587552) (width 0.25) (layer "F.Cu") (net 11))
 (segment (start 146.55009 121.528978) (end 155.077022 121.528978) (width 0.25) (layer "F.Cu") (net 11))
 (segment (start 130.81 119.634) (end 133.604 116.84) (width 0.25) (layer "F.Cu") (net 11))
 (segment (start 141.861112 116.84) (end 146.55009 121.528978) (width 0.25) (layer "F.Cu") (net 11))
 (segment (start 155.077022 121.528978) (end 157.226 119.38) (width 0.25) (layer "F.Cu") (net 11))
 (segment (start 135.636 117.348) (end 141.733408 117.348) (width 0.25) (layer "F.Cu") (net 13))
 (segment (start 156.659511 121.978489) (end 159.766 118.872) (width 0.25) (layer "F.Cu") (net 13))
 (segment (start 141.733408 117.348) (end 146.363897 121.978489) (width 0.25) (layer "F.Cu") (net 13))
 (segment (start 159.766 118.872) (end 159.766 117.587552) (width 0.25) (layer "F.Cu") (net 13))
 (segment (start 146.363897 121.978489) (end 156.659511 121.978489) (width 0.25) (layer "F.Cu") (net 13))
 (segment (start 133.35 119.634) (end 135.636 117.348) (width 0.25) (layer "F.Cu") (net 13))
 (segment (start 157.988 122.428) (end 161.529553 118.886447) (width 0.25) (layer "F.Cu") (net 14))
 (segment (start 135.89 119.634) (end 137.60951 117.91449) (width 0.25) (layer "F.Cu") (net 14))
 (segment (start 137.60951 117.91449) (end 141.664194 117.91449) (width 0.25) (layer "F.Cu") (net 14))
 (segment (start 141.664194 117.91449) (end 146.177704 122.428) (width 0.25) (layer "F.Cu") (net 14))
 (segment (start 161.529553 118.886447) (end 161.529553 115.824) (width 0.25) (layer "F.Cu") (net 14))
 (segment (start 146.177704 122.428) (end 157.988 122.428) (width 0.25) (layer "F.Cu") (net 14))
 (segment (start 141.478 118.364) (end 139.7 118.364) (width 0.25) (layer "F.Cu") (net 15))
 (segment (start 139.7 118.364) (end 138.43 119.634) (width 0.25) (layer "F.Cu") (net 15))
 (segment (start 163.576 115.316) (end 163.576 118.618) (width 0.25) (layer "F.Cu") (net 15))
 (segment (start 159.258 122.936) (end 146.05 122.936) (width 0.25) (layer "F.Cu") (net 15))
 (segment (start 146.05 122.936) (end 141.478 118.364) (width 0.25) (layer "F.Cu") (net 15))
 (segment (start 161.529553 114.554) (end 162.814 114.554) (width 0.25) (layer "F.Cu") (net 15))
 (segment (start 163.576 118.618) (end 159.258 122.936) (width 0.25) (layer "F.Cu") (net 15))
 (segment (start 162.814 114.554) (end 163.576 115.316) (width 0.25) (layer "F.Cu") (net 15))
 (segment (start 115.316 111.76) (end 144.018 111.76) (width 0.25) (layer "F.Cu") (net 32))
 (segment (start 107.95 104.394) (end 115.316 111.76) (width 0.25) (layer "F.Cu") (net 32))
 (segment (start 144.018 111.76) (end 145.034 110.744) (width 0.25) (layer "F.Cu") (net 32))
 (segment (start 145.034 110.744) (end 147.842448 110.744) (width 0.25) (layer "F.Cu") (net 32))
 (segment (start 145.796 123.444) (end 159.512 123.444) (width 0.25) (layer "F.Cu") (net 16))
 (segment (start 162.814 113.284) (end 161.529553 113.284) (width 0.25) (layer "F.Cu") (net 16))
 (segment (start 159.512 123.444) (end 164.084 118.872) (width 0.25) (layer "F.Cu") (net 16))
 (segment (start 164.084 118.872) (end 164.084 114.554) (width 0.25) (layer "F.Cu") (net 16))
 (segment (start 140.97 119.634) (end 141.986 119.634) (width 0.25) (layer "F.Cu") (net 16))
 (segment (start 141.986 119.634) (end 145.796 123.444) (width 0.25) (layer "F.Cu") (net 16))
 (segment (start 164.084 114.554) (end 162.814 113.284) (width 0.25) (layer "F.Cu") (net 16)))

